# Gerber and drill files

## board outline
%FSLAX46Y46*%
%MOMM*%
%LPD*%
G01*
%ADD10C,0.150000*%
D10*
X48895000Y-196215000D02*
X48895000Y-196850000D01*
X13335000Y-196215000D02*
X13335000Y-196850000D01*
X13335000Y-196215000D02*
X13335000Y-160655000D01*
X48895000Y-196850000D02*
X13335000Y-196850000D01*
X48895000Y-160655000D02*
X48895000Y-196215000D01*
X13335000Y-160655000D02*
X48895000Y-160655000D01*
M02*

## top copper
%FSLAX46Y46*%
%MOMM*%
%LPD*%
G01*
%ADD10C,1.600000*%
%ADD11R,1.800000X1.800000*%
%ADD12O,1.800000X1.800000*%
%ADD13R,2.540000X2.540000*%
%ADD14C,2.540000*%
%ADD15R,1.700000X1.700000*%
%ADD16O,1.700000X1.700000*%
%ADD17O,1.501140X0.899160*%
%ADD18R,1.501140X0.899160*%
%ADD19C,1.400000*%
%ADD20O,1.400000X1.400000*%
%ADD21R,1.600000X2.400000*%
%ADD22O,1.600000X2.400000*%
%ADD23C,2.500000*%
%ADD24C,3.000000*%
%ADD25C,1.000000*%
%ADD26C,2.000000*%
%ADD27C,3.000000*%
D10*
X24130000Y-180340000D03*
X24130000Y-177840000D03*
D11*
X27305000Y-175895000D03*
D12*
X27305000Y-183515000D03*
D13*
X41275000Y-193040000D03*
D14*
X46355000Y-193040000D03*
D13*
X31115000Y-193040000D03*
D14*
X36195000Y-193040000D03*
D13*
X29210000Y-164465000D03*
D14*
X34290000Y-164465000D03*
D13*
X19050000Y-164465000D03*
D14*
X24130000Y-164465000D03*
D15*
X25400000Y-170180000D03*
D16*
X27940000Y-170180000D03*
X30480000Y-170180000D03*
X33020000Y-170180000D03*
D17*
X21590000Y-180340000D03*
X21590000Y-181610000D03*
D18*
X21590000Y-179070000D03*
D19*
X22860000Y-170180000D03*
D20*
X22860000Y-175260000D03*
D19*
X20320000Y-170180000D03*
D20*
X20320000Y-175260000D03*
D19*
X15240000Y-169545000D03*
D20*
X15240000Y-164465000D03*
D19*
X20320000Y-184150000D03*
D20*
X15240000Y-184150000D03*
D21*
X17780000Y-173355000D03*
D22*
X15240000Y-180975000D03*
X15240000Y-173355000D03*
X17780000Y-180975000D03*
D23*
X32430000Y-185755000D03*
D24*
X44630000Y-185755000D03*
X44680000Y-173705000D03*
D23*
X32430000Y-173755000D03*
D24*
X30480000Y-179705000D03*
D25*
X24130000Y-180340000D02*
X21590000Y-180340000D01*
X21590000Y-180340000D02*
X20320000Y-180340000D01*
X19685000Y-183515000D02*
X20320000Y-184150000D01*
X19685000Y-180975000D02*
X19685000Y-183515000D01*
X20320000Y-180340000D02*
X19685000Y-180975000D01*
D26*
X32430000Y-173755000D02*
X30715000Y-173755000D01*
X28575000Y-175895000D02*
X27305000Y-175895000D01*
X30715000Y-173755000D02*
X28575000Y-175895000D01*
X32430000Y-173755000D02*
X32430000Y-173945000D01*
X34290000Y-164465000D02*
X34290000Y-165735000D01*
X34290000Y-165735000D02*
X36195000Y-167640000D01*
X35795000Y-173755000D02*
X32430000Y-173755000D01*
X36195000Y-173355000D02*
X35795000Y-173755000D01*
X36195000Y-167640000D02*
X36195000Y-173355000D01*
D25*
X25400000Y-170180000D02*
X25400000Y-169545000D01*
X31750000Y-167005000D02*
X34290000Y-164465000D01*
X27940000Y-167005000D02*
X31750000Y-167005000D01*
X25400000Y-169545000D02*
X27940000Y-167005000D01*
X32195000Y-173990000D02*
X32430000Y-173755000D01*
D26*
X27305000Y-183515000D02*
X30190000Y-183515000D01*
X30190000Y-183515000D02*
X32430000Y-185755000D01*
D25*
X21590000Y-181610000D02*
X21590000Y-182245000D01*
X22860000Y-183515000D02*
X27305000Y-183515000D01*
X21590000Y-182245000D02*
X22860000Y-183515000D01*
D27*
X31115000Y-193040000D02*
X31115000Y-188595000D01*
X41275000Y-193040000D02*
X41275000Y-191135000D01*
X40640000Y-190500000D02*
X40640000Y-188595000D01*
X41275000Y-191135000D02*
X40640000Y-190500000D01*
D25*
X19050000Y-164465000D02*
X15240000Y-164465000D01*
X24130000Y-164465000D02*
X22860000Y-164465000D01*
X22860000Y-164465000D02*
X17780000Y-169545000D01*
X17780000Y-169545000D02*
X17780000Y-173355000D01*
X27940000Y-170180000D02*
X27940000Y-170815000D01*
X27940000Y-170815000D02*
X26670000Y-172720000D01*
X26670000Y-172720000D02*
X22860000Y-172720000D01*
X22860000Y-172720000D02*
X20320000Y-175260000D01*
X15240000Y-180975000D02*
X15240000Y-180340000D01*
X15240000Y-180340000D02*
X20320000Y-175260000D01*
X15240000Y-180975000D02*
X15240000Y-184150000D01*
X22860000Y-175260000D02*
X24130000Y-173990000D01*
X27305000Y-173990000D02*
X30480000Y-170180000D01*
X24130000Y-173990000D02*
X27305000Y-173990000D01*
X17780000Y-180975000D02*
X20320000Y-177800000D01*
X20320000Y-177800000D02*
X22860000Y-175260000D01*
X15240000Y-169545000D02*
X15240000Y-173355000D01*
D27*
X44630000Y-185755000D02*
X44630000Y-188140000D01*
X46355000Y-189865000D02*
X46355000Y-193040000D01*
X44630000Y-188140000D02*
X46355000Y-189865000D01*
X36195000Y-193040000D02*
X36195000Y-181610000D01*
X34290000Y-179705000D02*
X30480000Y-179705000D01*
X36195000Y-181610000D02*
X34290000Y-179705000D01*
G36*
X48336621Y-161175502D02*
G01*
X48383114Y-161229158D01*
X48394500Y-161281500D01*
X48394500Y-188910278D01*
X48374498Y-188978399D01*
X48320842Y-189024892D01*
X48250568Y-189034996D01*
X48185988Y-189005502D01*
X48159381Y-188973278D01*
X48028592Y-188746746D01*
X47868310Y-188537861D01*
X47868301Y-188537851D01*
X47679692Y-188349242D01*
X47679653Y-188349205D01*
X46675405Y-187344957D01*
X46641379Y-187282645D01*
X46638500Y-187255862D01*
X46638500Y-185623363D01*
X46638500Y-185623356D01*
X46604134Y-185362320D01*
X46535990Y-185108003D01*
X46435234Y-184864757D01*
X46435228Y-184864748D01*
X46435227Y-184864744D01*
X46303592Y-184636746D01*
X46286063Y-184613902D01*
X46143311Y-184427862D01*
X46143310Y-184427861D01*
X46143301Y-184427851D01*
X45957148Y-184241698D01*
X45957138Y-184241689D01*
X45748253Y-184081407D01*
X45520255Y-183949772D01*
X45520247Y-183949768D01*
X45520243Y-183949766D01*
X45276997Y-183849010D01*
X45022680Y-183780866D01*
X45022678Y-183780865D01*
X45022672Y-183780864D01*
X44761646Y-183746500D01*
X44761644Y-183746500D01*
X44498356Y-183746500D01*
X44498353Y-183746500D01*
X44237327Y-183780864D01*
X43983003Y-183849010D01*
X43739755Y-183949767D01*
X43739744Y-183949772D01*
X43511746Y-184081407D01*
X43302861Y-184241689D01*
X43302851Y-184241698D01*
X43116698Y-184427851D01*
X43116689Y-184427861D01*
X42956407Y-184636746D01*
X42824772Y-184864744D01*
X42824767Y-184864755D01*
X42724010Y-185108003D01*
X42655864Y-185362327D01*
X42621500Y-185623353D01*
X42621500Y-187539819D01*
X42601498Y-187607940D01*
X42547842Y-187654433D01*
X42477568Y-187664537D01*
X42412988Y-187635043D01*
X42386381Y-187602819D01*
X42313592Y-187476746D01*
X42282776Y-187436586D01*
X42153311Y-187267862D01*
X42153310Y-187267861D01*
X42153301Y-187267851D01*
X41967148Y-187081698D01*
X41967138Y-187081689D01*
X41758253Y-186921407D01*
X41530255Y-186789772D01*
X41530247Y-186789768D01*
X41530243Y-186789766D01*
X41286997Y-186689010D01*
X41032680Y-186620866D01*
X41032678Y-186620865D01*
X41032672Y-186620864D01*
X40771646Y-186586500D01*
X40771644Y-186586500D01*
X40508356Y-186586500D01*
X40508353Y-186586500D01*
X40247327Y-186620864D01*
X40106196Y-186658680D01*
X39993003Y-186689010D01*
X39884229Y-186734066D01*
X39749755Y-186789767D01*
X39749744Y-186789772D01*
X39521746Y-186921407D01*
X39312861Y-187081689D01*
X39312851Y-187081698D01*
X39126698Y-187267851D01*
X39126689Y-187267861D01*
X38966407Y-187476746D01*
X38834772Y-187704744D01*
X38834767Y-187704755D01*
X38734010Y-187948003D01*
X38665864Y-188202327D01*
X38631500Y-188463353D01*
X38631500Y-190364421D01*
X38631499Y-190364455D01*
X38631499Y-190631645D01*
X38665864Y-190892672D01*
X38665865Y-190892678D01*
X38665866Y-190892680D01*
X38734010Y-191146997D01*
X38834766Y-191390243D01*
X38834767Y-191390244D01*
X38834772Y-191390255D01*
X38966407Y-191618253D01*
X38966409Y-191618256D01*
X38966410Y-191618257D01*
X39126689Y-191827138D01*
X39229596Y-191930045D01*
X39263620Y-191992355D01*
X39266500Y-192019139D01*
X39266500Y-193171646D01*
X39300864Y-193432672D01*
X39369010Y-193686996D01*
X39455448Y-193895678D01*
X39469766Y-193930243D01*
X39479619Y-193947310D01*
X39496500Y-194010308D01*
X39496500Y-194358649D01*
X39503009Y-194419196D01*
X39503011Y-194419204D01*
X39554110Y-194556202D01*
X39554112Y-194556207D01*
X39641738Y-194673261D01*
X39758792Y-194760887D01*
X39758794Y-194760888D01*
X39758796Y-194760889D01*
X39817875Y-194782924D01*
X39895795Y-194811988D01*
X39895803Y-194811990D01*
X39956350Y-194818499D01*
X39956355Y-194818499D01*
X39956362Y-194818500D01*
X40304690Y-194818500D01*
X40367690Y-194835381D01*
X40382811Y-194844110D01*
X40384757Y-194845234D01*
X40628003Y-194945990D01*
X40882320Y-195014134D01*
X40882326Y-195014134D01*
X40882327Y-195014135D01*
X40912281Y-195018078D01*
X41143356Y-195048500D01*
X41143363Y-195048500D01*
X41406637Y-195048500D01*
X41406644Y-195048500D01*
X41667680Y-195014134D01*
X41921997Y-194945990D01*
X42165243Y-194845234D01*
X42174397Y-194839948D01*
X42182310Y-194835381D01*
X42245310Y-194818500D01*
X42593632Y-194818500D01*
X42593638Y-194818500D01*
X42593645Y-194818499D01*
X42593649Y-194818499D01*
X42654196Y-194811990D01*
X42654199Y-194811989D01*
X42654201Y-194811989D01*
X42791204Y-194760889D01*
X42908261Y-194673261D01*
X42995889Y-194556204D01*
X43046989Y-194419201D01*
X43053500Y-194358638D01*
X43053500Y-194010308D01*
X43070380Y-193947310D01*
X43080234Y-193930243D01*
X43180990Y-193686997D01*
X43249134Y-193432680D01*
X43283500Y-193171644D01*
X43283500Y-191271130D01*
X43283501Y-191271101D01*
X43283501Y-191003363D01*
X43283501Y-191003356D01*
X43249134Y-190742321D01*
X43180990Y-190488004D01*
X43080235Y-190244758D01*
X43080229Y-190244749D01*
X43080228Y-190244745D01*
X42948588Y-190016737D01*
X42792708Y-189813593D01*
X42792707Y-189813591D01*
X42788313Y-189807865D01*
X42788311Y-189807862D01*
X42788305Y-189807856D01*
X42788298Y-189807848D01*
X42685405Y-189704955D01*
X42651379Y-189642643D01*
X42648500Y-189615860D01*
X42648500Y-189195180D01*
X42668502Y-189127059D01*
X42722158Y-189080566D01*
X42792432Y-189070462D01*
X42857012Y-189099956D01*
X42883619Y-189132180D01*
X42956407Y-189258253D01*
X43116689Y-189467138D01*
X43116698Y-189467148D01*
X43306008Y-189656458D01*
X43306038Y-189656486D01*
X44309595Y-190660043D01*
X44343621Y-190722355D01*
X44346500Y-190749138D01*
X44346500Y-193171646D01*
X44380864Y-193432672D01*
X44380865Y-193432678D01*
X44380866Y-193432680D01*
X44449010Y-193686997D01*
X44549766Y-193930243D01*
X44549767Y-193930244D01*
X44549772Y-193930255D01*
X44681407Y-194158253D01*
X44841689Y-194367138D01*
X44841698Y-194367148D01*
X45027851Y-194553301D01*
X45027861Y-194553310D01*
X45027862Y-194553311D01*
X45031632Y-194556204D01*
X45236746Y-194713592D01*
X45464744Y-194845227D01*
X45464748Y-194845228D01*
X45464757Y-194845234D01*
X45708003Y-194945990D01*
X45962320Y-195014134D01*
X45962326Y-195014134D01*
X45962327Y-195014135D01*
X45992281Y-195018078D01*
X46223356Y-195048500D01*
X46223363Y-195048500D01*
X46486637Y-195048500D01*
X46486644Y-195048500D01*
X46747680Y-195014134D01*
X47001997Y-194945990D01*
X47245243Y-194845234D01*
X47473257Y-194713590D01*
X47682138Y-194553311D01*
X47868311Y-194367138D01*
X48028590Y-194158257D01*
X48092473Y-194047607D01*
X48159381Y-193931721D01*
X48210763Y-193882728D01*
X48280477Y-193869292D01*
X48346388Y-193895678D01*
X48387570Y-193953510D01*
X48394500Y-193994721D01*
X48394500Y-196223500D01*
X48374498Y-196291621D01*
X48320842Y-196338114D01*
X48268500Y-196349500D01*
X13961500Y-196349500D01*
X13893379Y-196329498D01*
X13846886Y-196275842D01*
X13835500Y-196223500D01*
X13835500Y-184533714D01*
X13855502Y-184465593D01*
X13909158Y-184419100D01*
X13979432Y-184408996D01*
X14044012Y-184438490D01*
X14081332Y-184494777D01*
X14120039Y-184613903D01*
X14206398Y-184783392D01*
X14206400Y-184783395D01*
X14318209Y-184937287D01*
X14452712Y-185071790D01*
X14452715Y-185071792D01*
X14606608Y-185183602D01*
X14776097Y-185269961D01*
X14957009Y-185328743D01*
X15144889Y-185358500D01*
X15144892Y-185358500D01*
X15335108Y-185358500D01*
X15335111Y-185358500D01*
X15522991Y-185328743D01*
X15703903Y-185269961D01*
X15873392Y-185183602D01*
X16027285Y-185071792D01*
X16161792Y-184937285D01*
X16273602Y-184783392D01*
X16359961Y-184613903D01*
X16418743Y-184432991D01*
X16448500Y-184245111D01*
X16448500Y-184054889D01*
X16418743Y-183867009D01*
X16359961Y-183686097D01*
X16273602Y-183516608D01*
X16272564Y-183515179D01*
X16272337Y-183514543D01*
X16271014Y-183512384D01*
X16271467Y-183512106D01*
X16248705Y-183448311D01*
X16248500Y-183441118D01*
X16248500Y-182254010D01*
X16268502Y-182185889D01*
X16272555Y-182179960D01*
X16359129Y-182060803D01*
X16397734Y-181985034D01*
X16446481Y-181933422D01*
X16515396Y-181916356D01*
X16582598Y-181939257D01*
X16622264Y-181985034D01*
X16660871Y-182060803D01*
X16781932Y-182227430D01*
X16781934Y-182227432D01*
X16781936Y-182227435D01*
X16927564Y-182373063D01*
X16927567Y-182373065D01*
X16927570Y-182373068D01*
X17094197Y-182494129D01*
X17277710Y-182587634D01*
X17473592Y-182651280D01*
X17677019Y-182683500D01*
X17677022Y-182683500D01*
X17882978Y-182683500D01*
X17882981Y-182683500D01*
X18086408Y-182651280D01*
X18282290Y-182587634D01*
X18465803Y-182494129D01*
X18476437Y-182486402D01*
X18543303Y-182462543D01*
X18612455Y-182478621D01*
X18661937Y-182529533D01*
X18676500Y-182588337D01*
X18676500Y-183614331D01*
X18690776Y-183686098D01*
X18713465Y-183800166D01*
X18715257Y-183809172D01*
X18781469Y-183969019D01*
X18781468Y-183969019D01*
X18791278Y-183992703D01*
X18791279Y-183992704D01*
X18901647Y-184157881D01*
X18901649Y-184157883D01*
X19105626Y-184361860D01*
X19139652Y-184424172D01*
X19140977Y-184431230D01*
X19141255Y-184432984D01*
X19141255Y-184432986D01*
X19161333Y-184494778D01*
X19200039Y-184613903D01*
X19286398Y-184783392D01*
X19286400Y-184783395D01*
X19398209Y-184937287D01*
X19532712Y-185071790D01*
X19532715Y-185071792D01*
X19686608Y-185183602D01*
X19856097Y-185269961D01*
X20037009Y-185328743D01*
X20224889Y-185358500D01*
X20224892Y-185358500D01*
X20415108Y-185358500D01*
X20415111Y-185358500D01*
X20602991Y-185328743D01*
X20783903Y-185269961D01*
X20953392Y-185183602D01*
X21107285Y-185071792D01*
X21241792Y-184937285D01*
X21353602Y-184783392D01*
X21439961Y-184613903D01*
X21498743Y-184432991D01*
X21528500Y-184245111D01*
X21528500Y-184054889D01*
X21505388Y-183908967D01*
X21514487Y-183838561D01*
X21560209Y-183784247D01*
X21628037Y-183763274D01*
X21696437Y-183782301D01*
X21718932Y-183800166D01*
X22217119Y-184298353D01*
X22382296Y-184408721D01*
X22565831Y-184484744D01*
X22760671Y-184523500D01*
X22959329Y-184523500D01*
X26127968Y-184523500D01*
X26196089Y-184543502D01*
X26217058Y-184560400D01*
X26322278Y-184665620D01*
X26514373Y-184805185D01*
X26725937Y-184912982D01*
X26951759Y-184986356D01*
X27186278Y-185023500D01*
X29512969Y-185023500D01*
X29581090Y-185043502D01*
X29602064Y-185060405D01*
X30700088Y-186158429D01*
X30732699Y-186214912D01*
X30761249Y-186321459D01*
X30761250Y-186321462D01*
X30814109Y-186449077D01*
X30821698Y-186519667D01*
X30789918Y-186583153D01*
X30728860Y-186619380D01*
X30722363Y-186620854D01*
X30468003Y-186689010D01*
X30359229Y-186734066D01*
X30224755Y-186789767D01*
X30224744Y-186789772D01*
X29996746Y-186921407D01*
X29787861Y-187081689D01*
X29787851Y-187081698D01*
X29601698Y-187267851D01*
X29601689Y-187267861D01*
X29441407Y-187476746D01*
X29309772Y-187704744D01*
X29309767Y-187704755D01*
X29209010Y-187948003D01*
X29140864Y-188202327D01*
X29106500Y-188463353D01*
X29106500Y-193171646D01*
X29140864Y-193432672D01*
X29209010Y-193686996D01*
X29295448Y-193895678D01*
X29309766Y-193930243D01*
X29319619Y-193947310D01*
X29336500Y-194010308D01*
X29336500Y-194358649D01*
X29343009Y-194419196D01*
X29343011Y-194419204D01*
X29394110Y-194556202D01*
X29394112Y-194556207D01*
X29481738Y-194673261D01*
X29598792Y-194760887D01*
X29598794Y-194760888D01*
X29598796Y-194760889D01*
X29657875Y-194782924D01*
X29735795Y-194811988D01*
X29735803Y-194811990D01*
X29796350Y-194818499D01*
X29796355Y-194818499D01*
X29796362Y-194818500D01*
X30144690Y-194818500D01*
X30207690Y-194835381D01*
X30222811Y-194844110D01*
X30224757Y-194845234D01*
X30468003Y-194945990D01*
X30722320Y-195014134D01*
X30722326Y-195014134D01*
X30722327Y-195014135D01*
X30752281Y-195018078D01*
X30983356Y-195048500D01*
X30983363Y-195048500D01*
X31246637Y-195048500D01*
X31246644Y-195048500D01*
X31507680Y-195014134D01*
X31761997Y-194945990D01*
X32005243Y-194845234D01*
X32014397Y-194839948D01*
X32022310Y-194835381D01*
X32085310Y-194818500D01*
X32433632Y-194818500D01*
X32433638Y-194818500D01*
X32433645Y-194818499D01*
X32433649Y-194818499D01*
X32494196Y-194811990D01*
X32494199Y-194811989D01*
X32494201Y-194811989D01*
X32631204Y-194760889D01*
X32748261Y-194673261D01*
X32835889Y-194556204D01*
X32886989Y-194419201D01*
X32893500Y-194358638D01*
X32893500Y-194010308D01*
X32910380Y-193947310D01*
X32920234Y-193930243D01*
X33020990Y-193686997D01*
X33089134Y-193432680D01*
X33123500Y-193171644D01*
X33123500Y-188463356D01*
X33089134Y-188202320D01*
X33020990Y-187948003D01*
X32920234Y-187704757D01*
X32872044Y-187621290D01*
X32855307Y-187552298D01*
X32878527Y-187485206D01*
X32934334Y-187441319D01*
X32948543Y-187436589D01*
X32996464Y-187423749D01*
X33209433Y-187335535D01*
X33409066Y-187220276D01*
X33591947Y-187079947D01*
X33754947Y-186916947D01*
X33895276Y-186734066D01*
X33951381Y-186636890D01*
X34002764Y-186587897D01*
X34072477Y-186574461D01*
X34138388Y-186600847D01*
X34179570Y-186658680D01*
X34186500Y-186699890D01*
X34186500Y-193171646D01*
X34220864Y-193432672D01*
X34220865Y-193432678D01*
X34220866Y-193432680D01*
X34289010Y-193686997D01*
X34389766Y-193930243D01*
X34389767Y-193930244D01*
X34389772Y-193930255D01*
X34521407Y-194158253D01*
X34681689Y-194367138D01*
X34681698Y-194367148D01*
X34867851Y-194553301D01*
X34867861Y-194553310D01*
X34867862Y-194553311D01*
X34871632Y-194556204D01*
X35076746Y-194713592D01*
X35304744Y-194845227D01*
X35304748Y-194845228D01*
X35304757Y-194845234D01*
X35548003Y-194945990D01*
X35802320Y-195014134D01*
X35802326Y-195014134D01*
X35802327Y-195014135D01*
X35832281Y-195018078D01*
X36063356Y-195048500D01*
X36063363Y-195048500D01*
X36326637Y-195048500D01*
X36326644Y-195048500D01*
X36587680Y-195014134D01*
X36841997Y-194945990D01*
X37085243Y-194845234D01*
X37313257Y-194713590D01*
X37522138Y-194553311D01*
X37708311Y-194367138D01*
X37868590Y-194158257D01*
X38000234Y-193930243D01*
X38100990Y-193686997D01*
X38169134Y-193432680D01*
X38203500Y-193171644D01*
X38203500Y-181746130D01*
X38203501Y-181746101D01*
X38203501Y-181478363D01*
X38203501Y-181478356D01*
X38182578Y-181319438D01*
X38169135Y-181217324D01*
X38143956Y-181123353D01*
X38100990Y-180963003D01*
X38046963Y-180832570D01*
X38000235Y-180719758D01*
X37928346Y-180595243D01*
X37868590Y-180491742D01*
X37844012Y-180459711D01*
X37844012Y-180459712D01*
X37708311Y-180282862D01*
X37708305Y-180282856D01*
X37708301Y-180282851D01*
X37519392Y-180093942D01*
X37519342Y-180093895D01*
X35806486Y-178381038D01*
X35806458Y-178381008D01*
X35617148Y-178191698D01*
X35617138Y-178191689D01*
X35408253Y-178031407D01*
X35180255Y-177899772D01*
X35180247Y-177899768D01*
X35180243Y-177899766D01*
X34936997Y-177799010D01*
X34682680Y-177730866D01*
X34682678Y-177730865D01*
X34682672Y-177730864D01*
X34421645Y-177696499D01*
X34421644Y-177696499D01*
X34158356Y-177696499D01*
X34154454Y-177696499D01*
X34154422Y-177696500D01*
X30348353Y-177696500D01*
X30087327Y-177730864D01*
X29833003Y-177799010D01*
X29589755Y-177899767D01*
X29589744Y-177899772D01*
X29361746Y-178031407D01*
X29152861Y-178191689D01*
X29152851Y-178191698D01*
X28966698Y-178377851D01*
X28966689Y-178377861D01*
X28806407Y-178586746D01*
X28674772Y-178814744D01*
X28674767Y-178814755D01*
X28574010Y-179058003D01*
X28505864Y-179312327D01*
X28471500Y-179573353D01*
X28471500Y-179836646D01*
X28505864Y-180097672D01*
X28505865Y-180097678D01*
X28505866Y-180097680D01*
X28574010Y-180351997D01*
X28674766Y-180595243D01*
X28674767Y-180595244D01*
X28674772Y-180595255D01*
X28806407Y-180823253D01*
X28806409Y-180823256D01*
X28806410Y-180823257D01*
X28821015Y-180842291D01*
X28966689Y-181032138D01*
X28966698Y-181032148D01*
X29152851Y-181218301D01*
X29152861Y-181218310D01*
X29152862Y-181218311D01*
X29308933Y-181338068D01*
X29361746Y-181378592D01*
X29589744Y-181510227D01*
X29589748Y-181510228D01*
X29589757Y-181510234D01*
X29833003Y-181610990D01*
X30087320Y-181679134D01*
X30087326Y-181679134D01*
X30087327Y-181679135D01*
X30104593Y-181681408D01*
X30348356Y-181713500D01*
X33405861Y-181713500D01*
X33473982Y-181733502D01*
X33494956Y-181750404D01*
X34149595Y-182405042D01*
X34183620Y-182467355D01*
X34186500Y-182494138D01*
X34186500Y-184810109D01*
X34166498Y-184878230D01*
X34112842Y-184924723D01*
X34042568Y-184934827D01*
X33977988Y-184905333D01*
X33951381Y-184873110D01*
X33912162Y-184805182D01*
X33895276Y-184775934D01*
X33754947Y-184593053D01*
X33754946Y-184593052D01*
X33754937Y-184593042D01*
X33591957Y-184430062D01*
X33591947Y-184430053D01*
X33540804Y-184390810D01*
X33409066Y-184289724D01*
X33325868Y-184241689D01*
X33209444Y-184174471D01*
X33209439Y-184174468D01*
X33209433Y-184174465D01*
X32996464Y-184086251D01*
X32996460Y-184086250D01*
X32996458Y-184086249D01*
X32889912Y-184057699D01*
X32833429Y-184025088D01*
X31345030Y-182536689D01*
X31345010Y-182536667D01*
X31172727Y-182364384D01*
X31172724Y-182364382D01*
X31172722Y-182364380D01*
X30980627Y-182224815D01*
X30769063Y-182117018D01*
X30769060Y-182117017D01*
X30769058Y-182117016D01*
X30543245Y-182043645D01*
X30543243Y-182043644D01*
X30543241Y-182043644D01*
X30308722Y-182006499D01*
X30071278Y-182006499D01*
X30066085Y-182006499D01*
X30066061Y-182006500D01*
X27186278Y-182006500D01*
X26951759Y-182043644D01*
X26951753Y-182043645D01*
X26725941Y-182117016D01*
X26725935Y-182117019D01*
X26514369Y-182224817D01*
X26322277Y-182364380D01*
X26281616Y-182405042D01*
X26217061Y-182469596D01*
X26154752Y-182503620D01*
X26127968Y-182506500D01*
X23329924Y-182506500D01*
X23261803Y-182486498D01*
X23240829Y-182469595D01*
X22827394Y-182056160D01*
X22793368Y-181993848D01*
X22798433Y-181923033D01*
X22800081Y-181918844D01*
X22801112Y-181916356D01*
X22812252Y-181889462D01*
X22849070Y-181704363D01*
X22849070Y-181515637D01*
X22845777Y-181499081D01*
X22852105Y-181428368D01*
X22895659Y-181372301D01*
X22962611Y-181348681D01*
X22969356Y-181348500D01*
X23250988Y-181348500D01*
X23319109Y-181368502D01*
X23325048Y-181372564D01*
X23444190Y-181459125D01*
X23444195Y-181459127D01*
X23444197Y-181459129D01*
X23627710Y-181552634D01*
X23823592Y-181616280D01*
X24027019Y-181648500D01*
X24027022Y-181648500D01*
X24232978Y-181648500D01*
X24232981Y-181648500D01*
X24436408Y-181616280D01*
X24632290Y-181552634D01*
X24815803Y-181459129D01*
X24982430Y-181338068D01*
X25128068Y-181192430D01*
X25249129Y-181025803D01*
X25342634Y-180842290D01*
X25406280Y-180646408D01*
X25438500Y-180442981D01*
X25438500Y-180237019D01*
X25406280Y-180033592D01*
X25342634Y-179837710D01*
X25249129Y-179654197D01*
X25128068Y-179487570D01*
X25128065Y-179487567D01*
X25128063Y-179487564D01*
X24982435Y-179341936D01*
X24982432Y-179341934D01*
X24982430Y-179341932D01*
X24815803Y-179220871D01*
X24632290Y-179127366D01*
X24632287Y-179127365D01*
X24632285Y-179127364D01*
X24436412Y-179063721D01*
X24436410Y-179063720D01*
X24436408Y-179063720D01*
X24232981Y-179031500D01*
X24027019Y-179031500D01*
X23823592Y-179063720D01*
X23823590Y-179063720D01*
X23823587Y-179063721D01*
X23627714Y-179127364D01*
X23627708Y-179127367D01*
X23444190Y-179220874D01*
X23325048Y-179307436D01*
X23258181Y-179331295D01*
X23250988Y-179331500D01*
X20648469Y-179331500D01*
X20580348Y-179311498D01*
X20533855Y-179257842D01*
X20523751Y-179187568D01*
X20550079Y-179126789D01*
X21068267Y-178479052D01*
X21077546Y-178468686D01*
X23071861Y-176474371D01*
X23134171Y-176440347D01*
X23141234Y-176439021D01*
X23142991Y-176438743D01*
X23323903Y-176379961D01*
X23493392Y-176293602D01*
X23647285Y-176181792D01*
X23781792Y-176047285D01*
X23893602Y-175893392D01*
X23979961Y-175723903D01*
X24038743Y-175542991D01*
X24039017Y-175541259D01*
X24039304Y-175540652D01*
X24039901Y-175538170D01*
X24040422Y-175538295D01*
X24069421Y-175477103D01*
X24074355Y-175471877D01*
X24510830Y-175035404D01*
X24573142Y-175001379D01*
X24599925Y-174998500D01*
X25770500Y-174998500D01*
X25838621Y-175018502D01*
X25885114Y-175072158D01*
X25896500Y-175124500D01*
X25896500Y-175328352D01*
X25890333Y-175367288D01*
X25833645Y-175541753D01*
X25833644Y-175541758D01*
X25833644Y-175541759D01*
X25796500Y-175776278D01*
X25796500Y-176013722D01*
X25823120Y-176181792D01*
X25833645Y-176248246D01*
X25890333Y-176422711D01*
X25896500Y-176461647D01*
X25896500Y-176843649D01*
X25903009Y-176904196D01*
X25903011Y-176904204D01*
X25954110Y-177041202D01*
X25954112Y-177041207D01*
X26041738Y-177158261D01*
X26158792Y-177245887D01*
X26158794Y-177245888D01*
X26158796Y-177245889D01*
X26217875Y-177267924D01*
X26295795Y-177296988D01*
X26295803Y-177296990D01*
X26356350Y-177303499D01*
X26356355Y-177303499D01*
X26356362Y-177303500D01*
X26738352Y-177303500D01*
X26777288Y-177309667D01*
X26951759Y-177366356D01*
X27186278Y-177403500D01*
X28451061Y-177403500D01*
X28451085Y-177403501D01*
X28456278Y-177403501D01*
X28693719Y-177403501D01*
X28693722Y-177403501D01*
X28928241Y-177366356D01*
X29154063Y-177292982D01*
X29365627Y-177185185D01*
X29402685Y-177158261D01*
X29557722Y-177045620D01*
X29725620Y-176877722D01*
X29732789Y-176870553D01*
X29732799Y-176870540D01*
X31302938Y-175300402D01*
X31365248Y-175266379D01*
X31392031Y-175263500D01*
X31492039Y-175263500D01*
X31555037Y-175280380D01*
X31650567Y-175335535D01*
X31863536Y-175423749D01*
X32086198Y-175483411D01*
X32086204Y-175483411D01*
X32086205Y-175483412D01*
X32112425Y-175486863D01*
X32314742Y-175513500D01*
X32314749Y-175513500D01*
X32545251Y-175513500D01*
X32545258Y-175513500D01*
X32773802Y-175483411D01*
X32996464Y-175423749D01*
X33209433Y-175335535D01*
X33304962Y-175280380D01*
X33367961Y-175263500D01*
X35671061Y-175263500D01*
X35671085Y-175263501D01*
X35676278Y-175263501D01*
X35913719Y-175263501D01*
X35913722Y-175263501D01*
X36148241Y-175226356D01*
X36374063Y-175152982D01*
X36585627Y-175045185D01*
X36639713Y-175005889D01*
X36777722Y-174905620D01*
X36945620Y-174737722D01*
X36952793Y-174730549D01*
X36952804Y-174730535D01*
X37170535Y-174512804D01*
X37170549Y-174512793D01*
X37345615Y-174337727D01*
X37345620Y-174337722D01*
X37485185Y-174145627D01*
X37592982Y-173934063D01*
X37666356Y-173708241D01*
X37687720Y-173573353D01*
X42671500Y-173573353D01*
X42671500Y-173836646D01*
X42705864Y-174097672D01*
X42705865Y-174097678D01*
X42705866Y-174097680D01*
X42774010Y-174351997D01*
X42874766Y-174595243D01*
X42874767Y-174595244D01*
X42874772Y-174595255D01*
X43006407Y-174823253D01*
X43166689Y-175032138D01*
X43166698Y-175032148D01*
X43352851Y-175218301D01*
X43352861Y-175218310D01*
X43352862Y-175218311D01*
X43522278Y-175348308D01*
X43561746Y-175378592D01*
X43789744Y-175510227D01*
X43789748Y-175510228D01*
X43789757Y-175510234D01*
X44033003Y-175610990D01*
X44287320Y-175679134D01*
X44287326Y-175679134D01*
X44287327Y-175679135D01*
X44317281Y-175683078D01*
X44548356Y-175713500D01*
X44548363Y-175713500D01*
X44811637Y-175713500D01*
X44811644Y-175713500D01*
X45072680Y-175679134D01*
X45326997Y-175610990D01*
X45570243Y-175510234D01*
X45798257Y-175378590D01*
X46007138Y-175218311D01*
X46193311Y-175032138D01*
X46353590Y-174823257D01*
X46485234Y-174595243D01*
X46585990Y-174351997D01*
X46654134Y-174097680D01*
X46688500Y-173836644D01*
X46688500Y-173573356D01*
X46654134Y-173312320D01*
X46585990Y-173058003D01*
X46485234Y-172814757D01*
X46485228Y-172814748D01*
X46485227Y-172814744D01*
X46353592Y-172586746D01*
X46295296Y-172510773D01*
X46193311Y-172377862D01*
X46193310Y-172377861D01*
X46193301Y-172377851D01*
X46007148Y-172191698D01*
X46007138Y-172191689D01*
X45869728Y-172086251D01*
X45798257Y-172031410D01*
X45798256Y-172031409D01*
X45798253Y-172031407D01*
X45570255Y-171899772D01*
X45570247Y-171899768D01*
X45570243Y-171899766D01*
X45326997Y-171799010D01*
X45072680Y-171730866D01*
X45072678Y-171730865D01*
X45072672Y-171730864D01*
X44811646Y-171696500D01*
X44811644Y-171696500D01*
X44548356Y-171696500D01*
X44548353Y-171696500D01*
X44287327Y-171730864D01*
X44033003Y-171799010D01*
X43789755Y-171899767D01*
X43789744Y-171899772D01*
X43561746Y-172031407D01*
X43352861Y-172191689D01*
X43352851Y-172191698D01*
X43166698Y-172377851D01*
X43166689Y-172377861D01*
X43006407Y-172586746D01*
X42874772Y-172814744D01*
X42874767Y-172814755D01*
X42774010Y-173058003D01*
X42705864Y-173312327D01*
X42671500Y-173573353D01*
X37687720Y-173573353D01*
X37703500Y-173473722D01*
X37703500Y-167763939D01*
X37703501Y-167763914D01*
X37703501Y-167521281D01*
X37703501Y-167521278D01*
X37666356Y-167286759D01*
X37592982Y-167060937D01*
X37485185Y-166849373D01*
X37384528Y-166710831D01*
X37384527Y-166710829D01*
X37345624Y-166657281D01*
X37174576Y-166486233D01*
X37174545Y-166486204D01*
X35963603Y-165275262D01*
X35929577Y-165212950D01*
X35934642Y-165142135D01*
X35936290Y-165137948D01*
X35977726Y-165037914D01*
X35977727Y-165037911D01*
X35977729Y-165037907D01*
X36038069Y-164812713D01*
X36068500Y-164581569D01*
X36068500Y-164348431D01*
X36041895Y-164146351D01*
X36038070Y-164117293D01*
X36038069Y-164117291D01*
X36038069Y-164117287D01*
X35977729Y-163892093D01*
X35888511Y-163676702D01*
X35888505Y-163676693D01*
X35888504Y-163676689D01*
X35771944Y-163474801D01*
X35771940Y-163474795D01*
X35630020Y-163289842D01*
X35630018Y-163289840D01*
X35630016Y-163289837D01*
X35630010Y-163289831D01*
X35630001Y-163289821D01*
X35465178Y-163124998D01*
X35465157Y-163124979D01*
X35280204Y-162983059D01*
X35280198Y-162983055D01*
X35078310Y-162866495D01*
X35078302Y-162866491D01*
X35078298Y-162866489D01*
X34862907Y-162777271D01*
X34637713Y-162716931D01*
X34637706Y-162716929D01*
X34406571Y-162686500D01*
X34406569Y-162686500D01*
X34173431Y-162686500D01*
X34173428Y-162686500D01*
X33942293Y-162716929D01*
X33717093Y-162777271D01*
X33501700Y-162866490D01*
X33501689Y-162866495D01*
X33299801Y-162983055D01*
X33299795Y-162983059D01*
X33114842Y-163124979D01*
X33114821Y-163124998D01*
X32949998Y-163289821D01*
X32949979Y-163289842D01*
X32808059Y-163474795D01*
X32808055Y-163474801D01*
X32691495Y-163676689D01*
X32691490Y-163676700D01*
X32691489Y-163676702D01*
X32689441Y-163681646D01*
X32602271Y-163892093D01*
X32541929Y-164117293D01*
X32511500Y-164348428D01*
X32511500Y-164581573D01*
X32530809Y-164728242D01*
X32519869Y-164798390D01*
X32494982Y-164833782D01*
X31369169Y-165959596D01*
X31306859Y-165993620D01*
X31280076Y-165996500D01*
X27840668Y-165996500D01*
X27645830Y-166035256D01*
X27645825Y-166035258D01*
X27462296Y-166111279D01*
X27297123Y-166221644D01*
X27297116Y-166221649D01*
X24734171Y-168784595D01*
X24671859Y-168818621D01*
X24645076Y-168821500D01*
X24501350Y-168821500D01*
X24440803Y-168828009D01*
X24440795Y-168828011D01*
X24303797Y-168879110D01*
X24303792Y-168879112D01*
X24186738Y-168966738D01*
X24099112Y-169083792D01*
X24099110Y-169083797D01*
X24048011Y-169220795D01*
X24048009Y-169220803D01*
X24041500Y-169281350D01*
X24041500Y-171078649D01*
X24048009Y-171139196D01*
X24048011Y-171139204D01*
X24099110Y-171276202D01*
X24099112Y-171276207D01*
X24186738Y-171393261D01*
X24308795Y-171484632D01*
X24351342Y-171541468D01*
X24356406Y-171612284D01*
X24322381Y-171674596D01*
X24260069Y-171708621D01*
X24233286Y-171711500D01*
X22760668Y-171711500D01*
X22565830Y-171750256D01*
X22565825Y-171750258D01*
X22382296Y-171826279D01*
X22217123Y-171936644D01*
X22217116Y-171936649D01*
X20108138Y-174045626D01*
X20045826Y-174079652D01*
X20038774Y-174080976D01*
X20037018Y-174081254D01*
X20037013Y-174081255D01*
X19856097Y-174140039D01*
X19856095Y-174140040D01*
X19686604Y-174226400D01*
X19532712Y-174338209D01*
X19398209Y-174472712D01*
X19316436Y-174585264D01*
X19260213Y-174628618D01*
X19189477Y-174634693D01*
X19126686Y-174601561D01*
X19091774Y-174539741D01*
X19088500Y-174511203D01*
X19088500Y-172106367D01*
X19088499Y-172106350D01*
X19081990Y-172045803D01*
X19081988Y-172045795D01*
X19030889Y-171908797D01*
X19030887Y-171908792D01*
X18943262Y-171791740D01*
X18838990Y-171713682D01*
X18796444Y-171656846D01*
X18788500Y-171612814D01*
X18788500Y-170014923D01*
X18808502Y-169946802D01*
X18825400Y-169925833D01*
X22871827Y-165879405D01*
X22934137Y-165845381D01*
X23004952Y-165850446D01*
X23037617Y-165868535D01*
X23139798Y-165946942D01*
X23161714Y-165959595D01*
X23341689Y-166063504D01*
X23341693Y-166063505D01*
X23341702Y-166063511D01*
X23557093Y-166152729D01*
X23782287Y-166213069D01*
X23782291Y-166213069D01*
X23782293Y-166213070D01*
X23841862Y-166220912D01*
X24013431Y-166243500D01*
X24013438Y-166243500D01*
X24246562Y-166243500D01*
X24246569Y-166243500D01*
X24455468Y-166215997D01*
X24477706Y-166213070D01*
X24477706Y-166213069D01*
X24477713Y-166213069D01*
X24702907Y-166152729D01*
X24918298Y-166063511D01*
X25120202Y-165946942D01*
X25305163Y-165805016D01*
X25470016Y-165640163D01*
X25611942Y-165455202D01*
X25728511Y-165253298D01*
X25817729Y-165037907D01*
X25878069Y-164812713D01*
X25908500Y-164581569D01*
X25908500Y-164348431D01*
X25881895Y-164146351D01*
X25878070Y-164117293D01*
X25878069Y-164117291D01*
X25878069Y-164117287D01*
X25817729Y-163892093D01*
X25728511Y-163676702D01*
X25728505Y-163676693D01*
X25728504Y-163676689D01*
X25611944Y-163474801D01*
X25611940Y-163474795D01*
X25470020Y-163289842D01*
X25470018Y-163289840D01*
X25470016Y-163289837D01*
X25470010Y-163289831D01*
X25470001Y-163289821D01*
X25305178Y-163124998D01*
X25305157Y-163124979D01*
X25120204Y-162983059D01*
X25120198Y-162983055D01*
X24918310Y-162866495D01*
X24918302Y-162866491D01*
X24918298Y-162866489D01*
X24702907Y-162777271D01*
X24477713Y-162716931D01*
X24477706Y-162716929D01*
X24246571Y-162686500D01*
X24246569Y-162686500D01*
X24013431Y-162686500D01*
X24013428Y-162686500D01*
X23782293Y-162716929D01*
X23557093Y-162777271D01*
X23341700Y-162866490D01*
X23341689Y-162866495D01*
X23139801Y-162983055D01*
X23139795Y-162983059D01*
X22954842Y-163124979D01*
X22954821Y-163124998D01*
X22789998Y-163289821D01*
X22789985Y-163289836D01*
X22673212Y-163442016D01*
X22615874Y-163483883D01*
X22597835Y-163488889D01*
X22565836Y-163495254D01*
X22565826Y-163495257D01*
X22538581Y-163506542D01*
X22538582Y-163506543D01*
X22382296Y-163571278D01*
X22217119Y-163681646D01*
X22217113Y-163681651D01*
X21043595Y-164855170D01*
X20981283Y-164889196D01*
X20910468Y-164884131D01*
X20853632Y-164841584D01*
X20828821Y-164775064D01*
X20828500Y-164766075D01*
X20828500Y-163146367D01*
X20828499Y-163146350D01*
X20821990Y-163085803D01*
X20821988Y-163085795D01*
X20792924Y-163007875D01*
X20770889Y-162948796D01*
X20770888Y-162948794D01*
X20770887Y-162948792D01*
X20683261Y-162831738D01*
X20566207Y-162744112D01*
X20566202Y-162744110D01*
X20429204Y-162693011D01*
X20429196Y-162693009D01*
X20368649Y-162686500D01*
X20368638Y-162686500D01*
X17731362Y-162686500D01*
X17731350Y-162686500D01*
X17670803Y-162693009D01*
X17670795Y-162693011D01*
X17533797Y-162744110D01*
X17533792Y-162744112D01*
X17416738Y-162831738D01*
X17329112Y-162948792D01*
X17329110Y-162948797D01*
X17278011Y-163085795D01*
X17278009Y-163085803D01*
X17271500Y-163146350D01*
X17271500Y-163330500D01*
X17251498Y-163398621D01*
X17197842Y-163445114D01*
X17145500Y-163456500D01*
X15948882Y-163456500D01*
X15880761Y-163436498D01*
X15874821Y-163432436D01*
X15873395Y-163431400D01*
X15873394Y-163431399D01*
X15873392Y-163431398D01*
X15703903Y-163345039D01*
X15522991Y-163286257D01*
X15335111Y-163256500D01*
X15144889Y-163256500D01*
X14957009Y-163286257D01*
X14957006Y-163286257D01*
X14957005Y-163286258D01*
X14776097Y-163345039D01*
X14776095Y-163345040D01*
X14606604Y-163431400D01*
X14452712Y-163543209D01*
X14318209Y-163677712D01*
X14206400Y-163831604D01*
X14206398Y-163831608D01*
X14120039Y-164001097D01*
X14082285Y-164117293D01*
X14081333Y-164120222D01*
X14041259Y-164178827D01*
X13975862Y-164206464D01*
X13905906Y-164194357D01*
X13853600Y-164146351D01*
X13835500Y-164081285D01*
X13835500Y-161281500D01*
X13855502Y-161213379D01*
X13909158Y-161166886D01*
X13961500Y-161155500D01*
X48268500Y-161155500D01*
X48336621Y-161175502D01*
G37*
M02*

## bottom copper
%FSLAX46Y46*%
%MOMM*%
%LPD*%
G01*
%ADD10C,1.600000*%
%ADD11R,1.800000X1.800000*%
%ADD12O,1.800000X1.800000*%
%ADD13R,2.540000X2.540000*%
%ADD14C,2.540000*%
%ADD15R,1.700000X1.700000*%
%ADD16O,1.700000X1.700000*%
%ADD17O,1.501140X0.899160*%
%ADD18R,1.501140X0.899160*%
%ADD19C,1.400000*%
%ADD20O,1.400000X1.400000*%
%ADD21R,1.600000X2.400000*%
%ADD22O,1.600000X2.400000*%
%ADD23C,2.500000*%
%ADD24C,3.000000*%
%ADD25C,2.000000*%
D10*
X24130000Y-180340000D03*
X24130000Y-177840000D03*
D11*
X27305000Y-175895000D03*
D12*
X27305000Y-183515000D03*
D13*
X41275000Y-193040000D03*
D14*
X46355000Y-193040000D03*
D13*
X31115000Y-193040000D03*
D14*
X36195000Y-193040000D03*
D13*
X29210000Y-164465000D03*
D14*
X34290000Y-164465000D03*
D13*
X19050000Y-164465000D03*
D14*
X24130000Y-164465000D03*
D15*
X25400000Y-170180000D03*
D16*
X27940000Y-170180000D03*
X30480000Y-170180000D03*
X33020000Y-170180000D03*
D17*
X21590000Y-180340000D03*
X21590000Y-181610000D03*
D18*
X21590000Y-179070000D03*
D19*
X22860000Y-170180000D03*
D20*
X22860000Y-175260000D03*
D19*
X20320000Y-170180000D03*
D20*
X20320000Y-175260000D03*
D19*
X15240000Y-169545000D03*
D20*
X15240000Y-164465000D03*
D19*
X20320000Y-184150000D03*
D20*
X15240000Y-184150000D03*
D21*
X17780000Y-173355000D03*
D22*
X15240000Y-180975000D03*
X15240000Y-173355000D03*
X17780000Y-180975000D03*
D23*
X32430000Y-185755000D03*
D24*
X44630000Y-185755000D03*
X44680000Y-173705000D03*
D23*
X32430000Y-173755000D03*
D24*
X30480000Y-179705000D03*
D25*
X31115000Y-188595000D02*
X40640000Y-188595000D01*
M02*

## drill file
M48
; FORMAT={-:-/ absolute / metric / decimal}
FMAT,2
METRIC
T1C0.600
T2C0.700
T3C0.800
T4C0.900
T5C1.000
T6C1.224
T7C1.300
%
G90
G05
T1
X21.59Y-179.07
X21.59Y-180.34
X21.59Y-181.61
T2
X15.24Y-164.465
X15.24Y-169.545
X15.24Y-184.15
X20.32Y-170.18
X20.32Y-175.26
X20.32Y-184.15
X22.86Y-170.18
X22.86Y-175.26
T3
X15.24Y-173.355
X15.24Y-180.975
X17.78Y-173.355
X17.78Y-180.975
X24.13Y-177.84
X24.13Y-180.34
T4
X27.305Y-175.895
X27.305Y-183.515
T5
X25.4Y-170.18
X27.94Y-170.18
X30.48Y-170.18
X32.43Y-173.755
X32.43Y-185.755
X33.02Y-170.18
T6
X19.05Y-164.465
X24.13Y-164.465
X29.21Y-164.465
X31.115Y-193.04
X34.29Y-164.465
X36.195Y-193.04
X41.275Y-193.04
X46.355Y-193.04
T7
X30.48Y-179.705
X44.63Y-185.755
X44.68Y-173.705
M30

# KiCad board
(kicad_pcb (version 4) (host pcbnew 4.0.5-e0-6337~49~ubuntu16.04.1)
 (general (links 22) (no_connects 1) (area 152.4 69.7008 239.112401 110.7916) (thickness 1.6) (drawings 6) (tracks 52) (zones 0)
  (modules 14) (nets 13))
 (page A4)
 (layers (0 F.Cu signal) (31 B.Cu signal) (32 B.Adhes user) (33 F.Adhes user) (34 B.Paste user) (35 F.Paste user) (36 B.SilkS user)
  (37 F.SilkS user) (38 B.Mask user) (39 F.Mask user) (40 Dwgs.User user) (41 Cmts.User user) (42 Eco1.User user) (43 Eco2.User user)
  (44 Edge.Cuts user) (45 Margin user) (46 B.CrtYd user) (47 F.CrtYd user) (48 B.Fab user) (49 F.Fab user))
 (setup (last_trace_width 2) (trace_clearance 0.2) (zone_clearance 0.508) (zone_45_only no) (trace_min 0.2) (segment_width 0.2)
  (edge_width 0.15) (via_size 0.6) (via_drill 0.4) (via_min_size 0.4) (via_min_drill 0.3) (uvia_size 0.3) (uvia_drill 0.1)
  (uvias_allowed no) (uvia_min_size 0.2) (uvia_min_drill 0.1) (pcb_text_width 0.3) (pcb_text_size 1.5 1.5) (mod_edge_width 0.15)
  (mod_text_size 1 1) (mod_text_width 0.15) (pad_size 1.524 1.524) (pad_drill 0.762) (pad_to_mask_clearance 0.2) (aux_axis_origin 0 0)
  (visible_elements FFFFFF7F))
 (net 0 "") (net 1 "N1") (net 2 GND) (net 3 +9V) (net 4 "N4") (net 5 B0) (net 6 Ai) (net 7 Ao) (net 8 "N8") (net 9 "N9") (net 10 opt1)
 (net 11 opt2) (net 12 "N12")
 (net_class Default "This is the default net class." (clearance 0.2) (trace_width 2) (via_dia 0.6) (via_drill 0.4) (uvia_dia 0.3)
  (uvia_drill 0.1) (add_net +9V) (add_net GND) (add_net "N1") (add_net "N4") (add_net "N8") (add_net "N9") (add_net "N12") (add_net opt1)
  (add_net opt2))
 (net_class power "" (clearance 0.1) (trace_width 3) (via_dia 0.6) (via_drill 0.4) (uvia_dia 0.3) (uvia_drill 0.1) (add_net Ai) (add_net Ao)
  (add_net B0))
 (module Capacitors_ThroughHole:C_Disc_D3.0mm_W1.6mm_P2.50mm (layer F.Cu) (at 24.13 180.34 90)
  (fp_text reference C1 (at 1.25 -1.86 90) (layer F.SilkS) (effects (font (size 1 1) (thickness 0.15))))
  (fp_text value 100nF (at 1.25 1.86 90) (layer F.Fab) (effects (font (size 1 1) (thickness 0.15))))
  (pad 1 thru_hole circle (at 0 0 90) (size 1.6 1.6) (drill 0.8) (layers *.Cu *.Mask) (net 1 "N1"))
  (pad 2 thru_hole circle (at 2.5 0 90) (size 1.6 1.6) (drill 0.8) (layers *.Cu *.Mask) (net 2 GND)))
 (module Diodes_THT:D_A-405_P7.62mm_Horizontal (layer F.Cu) (at 27.305 175.895 270)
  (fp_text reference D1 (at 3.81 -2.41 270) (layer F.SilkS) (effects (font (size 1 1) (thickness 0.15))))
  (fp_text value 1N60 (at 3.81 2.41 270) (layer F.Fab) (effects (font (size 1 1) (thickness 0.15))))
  (pad 1 thru_hole rect (at 0 0 270) (size 1.8 1.8) (drill 0.9) (layers *.Cu *.Mask) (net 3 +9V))
  (pad 2 thru_hole oval (at 7.62 0 270) (size 1.8 1.8) (drill 0.9) (layers *.Cu *.Mask) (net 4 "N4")))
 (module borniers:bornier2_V (layer F.Cu) (at 43.815 193.04)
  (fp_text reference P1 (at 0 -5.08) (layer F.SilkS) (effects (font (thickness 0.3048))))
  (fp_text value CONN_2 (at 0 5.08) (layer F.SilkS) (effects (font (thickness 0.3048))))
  (pad 1 thru_hole rect (at -2.54 0) (size 2.54 2.54) (drill 1.22428) (layers *.Cu *.Mask F.SilkS) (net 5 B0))
  (pad 2 thru_hole circle (at 2.54 0) (size 2.54 2.54) (drill 1.22428) (layers *.Cu *.Mask F.SilkS) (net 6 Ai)))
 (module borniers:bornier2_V (layer F.Cu) (at 33.655 193.04)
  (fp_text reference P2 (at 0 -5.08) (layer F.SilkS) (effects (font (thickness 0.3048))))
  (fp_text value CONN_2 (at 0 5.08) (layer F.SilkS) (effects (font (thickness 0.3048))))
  (pad 1 thru_hole rect (at -2.54 0) (size 2.54 2.54) (drill 1.22428) (layers *.Cu *.Mask F.SilkS) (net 5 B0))
  (pad 2 thru_hole circle (at 2.54 0) (size 2.54 2.54) (drill 1.22428) (layers *.Cu *.Mask F.SilkS) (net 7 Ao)))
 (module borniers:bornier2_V (layer F.Cu) (at 31.75 164.465)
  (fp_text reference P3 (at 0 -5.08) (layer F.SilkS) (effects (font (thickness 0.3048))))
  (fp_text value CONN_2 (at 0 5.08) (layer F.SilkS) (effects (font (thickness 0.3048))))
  (pad 1 thru_hole rect (at -2.54 0) (size 2.54 2.54) (drill 1.22428) (layers *.Cu *.Mask F.SilkS) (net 2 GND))
  (pad 2 thru_hole circle (at 2.54 0) (size 2.54 2.54) (drill 1.22428) (layers *.Cu *.Mask F.SilkS) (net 3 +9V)))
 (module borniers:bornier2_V (layer F.Cu) (at 21.59 164.465)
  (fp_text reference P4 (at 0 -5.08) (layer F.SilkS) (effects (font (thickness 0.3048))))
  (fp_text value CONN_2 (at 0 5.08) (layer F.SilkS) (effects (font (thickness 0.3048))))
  (pad 1 thru_hole rect (at -2.54 0) (size 2.54 2.54) (drill 1.22428) (layers *.Cu *.Mask F.SilkS) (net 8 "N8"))
  (pad 2 thru_hole circle (at 2.54 0) (size 2.54 2.54) (drill 1.22428) (layers *.Cu *.Mask F.SilkS) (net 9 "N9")))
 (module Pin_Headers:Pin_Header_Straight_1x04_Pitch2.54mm (layer F.Cu) (at 25.4 170.18 90)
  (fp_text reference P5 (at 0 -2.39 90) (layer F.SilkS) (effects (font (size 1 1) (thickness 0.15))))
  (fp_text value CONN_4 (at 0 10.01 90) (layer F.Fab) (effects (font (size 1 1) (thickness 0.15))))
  (pad 1 thru_hole rect (at 0 0 90) (size 1.7 1.7) (drill 1) (layers *.Cu *.Mask) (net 3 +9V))
  (pad 2 thru_hole oval (at 0 2.54 90) (size 1.7 1.7) (drill 1) (layers *.Cu *.Mask) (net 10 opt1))
  (pad 3 thru_hole oval (at 0 5.08 90) (size 1.7 1.7) (drill 1) (layers *.Cu *.Mask) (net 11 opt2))
  (pad 4 thru_hole oval (at 0 7.62 90) (size 1.7 1.7) (drill 1) (layers *.Cu *.Mask)))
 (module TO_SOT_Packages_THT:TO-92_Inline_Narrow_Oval (layer F.Cu) (at 21.59 179.07 270)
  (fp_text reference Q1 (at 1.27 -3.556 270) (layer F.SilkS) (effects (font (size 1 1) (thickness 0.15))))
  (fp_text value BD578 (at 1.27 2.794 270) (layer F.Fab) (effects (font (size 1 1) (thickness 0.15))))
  (pad 2 thru_hole oval (at 1.27 0 90) (size 0.89916 1.50114) (drill 0.6) (layers *.Cu *.Mask) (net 1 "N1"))
  (pad 3 thru_hole oval (at 2.54 0 90) (size 0.89916 1.50114) (drill 0.6) (layers *.Cu *.Mask) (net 4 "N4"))
  (pad 1 thru_hole rect (at 0 0 90) (size 0.89916 1.50114) (drill 0.6) (layers *.Cu *.Mask) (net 2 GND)))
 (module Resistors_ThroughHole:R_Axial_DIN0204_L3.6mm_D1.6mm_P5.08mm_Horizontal (layer F.Cu) (at 22.86 170.18 270)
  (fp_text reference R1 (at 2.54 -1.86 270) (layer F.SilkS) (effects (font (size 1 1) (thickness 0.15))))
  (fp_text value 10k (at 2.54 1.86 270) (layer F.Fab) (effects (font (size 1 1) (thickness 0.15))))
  (pad 1 thru_hole circle (at 0 0 270) (size 1.4 1.4) (drill 0.7) (layers *.Cu *.Mask) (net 2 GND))
  (pad 2 thru_hole oval (at 5.08 0 270) (size 1.4 1.4) (drill 0.7) (layers *.Cu *.Mask) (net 11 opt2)))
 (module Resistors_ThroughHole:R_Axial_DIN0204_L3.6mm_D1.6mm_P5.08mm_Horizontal (layer F.Cu) (at 20.32 170.18 270)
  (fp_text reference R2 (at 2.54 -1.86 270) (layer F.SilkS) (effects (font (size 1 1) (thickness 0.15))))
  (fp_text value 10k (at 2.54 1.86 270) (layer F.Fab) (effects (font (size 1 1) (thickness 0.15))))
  (pad 1 thru_hole circle (at 0 0 270) (size 1.4 1.4) (drill 0.7) (layers *.Cu *.Mask) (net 2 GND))
  (pad 2 thru_hole oval (at 5.08 0 270) (size 1.4 1.4) (drill 0.7) (layers *.Cu *.Mask) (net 10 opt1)))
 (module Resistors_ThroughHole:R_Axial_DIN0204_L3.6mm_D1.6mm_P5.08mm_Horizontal (layer F.Cu) (at 15.24 169.545 90)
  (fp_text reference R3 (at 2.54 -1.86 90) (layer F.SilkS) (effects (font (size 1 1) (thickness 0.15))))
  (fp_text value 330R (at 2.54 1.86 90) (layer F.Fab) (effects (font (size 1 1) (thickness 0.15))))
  (pad 1 thru_hole circle (at 0 0 90) (size 1.4 1.4) (drill 0.7) (layers *.Cu *.Mask) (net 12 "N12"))
  (pad 2 thru_hole oval (at 5.08 0 90) (size 1.4 1.4) (drill 0.7) (layers *.Cu *.Mask) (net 8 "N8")))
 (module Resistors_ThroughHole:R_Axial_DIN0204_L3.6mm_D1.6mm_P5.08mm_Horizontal (layer F.Cu) (at 20.32 184.15 180)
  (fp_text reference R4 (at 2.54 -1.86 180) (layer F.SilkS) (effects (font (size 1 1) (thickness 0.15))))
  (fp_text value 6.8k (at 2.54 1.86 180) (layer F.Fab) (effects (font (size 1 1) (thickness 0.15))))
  (pad 1 thru_hole circle (at 0 0 180) (size 1.4 1.4) (drill 0.7) (layers *.Cu *.Mask) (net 1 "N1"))
  (pad 2 thru_hole oval (at 5.08 0 180) (size 1.4 1.4) (drill 0.7) (layers *.Cu *.Mask) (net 10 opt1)))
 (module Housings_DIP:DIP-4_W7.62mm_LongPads (layer F.Cu) (at 17.78 173.355 270)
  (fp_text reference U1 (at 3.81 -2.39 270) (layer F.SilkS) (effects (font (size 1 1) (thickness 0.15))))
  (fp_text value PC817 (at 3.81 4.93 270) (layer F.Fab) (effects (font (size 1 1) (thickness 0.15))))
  (pad 1 thru_hole rect (at 0 0 270) (size 2.4 1.6) (drill 0.8) (layers *.Cu *.Mask) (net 9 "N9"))
  (pad 3 thru_hole oval (at 7.62 2.54 270) (size 2.4 1.6) (drill 0.8) (layers *.Cu *.Mask) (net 10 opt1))
  (pad 2 thru_hole oval (at 0 2.54 270) (size 2.4 1.6) (drill 0.8) (layers *.Cu *.Mask) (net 12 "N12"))
  (pad 4 thru_hole oval (at 7.62 0 270) (size 2.4 1.6) (drill 0.8) (layers *.Cu *.Mask) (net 11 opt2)))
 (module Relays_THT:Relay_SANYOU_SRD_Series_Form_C (layer F.Cu) (at 30.48 179.705)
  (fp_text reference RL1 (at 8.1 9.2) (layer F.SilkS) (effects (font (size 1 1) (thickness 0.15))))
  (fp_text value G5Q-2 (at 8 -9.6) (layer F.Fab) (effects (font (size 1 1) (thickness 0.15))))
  (pad 2 thru_hole circle (at 1.95 6.05 90) (size 2.5 2.5) (drill 1) (layers *.Cu *.Mask) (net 4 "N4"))
  (pad 3 thru_hole circle (at 14.15 6.05 90) (size 3 3) (drill 1.3) (layers *.Cu *.Mask) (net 6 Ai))
  (pad 4 thru_hole circle (at 14.2 -6 90) (size 3 3) (drill 1.3) (layers *.Cu *.Mask))
  (pad 5 thru_hole circle (at 1.95 -5.95 90) (size 2.5 2.5) (drill 1) (layers *.Cu *.Mask) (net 3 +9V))
  (pad 1 thru_hole circle (at 0 0 90) (size 3 3) (drill 1.3) (layers *.Cu *.Mask) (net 7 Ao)))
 (gr_line (start 48.895 196.215) (end 48.895 196.85) (angle 90) (layer Edge.Cuts) (width 0.15))
 (gr_line (start 13.335 196.215) (end 13.335 196.85) (angle 90) (layer Edge.Cuts) (width 0.15))
 (gr_line (start 13.335 196.215) (end 13.335 160.655) (angle 90) (layer Edge.Cuts) (width 0.15))
 (gr_line (start 48.895 196.85) (end 13.335 196.85) (angle 90) (layer Edge.Cuts) (width 0.15))
 (gr_line (start 48.895 160.655) (end 48.895 196.215) (angle 90) (layer Edge.Cuts) (width 0.15))
 (gr_line (start 13.335 160.655) (end 48.895 160.655) (angle 90) (layer Edge.Cuts) (width 0.15))
 (segment (start 31.115 188.595) (end 40.64 188.595) (width 2) (layer B.Cu) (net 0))
 (segment (start 24.13 180.34) (end 21.59 180.34) (width 1) (layer F.Cu) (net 1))
 (segment (start 21.59 180.34) (end 20.32 180.34) (width 1) (layer F.Cu) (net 1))
 (segment (start 19.685 183.515) (end 20.32 184.15) (width 1) (layer F.Cu) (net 1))
 (segment (start 19.685 180.975) (end 19.685 183.515) (width 1) (layer F.Cu) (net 1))
 (segment (start 20.32 180.34) (end 19.685 180.975) (width 1) (layer F.Cu) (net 1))
 (segment (start 32.43 173.755) (end 30.715 173.755) (width 2) (layer F.Cu) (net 3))
 (segment (start 28.575 175.895) (end 27.305 175.895) (width 2) (layer F.Cu) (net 3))
 (segment (start 30.715 173.755) (end 28.575 175.895) (width 2) (layer F.Cu) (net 3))
 (segment (start 32.43 173.755) (end 32.43 173.945) (width 2) (layer F.Cu) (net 3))
 (segment (start 34.29 164.465) (end 34.29 165.735) (width 2) (layer F.Cu) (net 3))
 (segment (start 34.29 165.735) (end 36.195 167.64) (width 2) (layer F.Cu) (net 3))
 (segment (start 35.795 173.755) (end 32.43 173.755) (width 2) (layer F.Cu) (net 3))
 (segment (start 36.195 173.355) (end 35.795 173.755) (width 2) (layer F.Cu) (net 3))
 (segment (start 36.195 167.64) (end 36.195 173.355) (width 2) (layer F.Cu) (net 3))
 (segment (start 25.4 170.18) (end 25.4 169.545) (width 1) (layer F.Cu) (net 3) (status 10))
 (segment (start 31.75 167.005) (end 34.29 164.465) (width 1) (layer F.Cu) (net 3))
 (segment (start 27.94 167.005) (end 31.75 167.005) (width 1) (layer F.Cu) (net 3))
 (segment (start 25.4 169.545) (end 27.94 167.005) (width 1) (layer F.Cu) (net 3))
 (segment (start 32.195 173.99) (end 32.43 173.755) (width 1) (layer F.Cu) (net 3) (status 30))
 (segment (start 27.305 183.515) (end 30.19 183.515) (width 2) (layer F.Cu) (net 4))
 (segment (start 30.19 183.515) (end 32.43 185.755) (width 2) (layer F.Cu) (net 4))
 (segment (start 21.59 181.61) (end 21.59 182.245) (width 1) (layer F.Cu) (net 4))
 (segment (start 22.86 183.515) (end 27.305 183.515) (width 1) (layer F.Cu) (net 4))
 (segment (start 21.59 182.245) (end 22.86 183.515) (width 1) (layer F.Cu) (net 4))
 (segment (start 31.115 193.04) (end 31.115 188.595) (width 3) (layer F.Cu) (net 5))
 (segment (start 41.275 193.04) (end 41.275 191.135) (width 3) (layer F.Cu) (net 5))
 (segment (start 40.64 190.5) (end 40.64 188.595) (width 3) (layer F.Cu) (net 5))
 (segment (start 41.275 191.135) (end 40.64 190.5) (width 3) (layer F.Cu) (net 5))
 (segment (start 19.05 164.465) (end 15.24 164.465) (width 1) (layer F.Cu) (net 8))
 (segment (start 24.13 164.465) (end 22.86 164.465) (width 1) (layer F.Cu) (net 9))
 (segment (start 22.86 164.465) (end 17.78 169.545) (width 1) (layer F.Cu) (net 9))
 (segment (start 17.78 169.545) (end 17.78 173.355) (width 1) (layer F.Cu) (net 9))
 (segment (start 27.94 170.18) (end 27.94 170.815) (width 1) (layer F.Cu) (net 10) (status 30))
 (segment (start 27.94 170.815) (end 26.67 172.72) (width 1) (layer F.Cu) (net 10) (status 10))
 (segment (start 26.67 172.72) (end 22.86 172.72) (width 1) (layer F.Cu) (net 10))
 (segment (start 22.86 172.72) (end 20.32 175.26) (width 1) (layer F.Cu) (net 10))
 (segment (start 15.24 180.975) (end 15.24 180.34) (width 1) (layer F.Cu) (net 10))
 (segment (start 15.24 180.34) (end 20.32 175.26) (width 1) (layer F.Cu) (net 10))
 (segment (start 15.24 180.975) (end 15.24 184.15) (width 1) (layer F.Cu) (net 10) (status 10))
 (segment (start 22.86 175.26) (end 24.13 173.99) (width 1) (layer F.Cu) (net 11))
 (segment (start 27.305 173.99) (end 30.48 170.18) (width 1) (layer F.Cu) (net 11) (status 20))
 (segment (start 24.13 173.99) (end 27.305 173.99) (width 1) (layer F.Cu) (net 11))
 (segment (start 17.78 180.975) (end 20.32 177.8) (width 1) (layer F.Cu) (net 11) (status 10))
 (segment (start 20.32 177.8) (end 22.86 175.26) (width 1) (layer F.Cu) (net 11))
 (segment (start 15.24 169.545) (end 15.24 173.355) (width 1) (layer F.Cu) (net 12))
 (segment (start 44.63 185.755) (end 44.63 188.14) (width 3) (layer F.Cu) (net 6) (status 10))
 (segment (start 46.355 189.865) (end 46.355 193.04) (width 3) (layer F.Cu) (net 6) (status 20))
 (segment (start 44.63 188.14) (end 46.355 189.865) (width 3) (layer F.Cu) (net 6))
 (segment (start 36.195 193.04) (end 36.195 181.61) (width 3) (layer F.Cu) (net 7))
 (segment (start 34.29 179.705) (end 30.48 179.705) (width 3) (layer F.Cu) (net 7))
 (segment (start 36.195 181.61) (end 34.29 179.705) (width 3) (layer F.Cu) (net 7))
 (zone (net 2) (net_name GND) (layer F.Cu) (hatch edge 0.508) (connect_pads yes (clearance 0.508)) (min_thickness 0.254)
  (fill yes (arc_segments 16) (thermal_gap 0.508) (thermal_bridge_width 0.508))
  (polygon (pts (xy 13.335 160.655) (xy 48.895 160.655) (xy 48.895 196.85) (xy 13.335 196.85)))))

